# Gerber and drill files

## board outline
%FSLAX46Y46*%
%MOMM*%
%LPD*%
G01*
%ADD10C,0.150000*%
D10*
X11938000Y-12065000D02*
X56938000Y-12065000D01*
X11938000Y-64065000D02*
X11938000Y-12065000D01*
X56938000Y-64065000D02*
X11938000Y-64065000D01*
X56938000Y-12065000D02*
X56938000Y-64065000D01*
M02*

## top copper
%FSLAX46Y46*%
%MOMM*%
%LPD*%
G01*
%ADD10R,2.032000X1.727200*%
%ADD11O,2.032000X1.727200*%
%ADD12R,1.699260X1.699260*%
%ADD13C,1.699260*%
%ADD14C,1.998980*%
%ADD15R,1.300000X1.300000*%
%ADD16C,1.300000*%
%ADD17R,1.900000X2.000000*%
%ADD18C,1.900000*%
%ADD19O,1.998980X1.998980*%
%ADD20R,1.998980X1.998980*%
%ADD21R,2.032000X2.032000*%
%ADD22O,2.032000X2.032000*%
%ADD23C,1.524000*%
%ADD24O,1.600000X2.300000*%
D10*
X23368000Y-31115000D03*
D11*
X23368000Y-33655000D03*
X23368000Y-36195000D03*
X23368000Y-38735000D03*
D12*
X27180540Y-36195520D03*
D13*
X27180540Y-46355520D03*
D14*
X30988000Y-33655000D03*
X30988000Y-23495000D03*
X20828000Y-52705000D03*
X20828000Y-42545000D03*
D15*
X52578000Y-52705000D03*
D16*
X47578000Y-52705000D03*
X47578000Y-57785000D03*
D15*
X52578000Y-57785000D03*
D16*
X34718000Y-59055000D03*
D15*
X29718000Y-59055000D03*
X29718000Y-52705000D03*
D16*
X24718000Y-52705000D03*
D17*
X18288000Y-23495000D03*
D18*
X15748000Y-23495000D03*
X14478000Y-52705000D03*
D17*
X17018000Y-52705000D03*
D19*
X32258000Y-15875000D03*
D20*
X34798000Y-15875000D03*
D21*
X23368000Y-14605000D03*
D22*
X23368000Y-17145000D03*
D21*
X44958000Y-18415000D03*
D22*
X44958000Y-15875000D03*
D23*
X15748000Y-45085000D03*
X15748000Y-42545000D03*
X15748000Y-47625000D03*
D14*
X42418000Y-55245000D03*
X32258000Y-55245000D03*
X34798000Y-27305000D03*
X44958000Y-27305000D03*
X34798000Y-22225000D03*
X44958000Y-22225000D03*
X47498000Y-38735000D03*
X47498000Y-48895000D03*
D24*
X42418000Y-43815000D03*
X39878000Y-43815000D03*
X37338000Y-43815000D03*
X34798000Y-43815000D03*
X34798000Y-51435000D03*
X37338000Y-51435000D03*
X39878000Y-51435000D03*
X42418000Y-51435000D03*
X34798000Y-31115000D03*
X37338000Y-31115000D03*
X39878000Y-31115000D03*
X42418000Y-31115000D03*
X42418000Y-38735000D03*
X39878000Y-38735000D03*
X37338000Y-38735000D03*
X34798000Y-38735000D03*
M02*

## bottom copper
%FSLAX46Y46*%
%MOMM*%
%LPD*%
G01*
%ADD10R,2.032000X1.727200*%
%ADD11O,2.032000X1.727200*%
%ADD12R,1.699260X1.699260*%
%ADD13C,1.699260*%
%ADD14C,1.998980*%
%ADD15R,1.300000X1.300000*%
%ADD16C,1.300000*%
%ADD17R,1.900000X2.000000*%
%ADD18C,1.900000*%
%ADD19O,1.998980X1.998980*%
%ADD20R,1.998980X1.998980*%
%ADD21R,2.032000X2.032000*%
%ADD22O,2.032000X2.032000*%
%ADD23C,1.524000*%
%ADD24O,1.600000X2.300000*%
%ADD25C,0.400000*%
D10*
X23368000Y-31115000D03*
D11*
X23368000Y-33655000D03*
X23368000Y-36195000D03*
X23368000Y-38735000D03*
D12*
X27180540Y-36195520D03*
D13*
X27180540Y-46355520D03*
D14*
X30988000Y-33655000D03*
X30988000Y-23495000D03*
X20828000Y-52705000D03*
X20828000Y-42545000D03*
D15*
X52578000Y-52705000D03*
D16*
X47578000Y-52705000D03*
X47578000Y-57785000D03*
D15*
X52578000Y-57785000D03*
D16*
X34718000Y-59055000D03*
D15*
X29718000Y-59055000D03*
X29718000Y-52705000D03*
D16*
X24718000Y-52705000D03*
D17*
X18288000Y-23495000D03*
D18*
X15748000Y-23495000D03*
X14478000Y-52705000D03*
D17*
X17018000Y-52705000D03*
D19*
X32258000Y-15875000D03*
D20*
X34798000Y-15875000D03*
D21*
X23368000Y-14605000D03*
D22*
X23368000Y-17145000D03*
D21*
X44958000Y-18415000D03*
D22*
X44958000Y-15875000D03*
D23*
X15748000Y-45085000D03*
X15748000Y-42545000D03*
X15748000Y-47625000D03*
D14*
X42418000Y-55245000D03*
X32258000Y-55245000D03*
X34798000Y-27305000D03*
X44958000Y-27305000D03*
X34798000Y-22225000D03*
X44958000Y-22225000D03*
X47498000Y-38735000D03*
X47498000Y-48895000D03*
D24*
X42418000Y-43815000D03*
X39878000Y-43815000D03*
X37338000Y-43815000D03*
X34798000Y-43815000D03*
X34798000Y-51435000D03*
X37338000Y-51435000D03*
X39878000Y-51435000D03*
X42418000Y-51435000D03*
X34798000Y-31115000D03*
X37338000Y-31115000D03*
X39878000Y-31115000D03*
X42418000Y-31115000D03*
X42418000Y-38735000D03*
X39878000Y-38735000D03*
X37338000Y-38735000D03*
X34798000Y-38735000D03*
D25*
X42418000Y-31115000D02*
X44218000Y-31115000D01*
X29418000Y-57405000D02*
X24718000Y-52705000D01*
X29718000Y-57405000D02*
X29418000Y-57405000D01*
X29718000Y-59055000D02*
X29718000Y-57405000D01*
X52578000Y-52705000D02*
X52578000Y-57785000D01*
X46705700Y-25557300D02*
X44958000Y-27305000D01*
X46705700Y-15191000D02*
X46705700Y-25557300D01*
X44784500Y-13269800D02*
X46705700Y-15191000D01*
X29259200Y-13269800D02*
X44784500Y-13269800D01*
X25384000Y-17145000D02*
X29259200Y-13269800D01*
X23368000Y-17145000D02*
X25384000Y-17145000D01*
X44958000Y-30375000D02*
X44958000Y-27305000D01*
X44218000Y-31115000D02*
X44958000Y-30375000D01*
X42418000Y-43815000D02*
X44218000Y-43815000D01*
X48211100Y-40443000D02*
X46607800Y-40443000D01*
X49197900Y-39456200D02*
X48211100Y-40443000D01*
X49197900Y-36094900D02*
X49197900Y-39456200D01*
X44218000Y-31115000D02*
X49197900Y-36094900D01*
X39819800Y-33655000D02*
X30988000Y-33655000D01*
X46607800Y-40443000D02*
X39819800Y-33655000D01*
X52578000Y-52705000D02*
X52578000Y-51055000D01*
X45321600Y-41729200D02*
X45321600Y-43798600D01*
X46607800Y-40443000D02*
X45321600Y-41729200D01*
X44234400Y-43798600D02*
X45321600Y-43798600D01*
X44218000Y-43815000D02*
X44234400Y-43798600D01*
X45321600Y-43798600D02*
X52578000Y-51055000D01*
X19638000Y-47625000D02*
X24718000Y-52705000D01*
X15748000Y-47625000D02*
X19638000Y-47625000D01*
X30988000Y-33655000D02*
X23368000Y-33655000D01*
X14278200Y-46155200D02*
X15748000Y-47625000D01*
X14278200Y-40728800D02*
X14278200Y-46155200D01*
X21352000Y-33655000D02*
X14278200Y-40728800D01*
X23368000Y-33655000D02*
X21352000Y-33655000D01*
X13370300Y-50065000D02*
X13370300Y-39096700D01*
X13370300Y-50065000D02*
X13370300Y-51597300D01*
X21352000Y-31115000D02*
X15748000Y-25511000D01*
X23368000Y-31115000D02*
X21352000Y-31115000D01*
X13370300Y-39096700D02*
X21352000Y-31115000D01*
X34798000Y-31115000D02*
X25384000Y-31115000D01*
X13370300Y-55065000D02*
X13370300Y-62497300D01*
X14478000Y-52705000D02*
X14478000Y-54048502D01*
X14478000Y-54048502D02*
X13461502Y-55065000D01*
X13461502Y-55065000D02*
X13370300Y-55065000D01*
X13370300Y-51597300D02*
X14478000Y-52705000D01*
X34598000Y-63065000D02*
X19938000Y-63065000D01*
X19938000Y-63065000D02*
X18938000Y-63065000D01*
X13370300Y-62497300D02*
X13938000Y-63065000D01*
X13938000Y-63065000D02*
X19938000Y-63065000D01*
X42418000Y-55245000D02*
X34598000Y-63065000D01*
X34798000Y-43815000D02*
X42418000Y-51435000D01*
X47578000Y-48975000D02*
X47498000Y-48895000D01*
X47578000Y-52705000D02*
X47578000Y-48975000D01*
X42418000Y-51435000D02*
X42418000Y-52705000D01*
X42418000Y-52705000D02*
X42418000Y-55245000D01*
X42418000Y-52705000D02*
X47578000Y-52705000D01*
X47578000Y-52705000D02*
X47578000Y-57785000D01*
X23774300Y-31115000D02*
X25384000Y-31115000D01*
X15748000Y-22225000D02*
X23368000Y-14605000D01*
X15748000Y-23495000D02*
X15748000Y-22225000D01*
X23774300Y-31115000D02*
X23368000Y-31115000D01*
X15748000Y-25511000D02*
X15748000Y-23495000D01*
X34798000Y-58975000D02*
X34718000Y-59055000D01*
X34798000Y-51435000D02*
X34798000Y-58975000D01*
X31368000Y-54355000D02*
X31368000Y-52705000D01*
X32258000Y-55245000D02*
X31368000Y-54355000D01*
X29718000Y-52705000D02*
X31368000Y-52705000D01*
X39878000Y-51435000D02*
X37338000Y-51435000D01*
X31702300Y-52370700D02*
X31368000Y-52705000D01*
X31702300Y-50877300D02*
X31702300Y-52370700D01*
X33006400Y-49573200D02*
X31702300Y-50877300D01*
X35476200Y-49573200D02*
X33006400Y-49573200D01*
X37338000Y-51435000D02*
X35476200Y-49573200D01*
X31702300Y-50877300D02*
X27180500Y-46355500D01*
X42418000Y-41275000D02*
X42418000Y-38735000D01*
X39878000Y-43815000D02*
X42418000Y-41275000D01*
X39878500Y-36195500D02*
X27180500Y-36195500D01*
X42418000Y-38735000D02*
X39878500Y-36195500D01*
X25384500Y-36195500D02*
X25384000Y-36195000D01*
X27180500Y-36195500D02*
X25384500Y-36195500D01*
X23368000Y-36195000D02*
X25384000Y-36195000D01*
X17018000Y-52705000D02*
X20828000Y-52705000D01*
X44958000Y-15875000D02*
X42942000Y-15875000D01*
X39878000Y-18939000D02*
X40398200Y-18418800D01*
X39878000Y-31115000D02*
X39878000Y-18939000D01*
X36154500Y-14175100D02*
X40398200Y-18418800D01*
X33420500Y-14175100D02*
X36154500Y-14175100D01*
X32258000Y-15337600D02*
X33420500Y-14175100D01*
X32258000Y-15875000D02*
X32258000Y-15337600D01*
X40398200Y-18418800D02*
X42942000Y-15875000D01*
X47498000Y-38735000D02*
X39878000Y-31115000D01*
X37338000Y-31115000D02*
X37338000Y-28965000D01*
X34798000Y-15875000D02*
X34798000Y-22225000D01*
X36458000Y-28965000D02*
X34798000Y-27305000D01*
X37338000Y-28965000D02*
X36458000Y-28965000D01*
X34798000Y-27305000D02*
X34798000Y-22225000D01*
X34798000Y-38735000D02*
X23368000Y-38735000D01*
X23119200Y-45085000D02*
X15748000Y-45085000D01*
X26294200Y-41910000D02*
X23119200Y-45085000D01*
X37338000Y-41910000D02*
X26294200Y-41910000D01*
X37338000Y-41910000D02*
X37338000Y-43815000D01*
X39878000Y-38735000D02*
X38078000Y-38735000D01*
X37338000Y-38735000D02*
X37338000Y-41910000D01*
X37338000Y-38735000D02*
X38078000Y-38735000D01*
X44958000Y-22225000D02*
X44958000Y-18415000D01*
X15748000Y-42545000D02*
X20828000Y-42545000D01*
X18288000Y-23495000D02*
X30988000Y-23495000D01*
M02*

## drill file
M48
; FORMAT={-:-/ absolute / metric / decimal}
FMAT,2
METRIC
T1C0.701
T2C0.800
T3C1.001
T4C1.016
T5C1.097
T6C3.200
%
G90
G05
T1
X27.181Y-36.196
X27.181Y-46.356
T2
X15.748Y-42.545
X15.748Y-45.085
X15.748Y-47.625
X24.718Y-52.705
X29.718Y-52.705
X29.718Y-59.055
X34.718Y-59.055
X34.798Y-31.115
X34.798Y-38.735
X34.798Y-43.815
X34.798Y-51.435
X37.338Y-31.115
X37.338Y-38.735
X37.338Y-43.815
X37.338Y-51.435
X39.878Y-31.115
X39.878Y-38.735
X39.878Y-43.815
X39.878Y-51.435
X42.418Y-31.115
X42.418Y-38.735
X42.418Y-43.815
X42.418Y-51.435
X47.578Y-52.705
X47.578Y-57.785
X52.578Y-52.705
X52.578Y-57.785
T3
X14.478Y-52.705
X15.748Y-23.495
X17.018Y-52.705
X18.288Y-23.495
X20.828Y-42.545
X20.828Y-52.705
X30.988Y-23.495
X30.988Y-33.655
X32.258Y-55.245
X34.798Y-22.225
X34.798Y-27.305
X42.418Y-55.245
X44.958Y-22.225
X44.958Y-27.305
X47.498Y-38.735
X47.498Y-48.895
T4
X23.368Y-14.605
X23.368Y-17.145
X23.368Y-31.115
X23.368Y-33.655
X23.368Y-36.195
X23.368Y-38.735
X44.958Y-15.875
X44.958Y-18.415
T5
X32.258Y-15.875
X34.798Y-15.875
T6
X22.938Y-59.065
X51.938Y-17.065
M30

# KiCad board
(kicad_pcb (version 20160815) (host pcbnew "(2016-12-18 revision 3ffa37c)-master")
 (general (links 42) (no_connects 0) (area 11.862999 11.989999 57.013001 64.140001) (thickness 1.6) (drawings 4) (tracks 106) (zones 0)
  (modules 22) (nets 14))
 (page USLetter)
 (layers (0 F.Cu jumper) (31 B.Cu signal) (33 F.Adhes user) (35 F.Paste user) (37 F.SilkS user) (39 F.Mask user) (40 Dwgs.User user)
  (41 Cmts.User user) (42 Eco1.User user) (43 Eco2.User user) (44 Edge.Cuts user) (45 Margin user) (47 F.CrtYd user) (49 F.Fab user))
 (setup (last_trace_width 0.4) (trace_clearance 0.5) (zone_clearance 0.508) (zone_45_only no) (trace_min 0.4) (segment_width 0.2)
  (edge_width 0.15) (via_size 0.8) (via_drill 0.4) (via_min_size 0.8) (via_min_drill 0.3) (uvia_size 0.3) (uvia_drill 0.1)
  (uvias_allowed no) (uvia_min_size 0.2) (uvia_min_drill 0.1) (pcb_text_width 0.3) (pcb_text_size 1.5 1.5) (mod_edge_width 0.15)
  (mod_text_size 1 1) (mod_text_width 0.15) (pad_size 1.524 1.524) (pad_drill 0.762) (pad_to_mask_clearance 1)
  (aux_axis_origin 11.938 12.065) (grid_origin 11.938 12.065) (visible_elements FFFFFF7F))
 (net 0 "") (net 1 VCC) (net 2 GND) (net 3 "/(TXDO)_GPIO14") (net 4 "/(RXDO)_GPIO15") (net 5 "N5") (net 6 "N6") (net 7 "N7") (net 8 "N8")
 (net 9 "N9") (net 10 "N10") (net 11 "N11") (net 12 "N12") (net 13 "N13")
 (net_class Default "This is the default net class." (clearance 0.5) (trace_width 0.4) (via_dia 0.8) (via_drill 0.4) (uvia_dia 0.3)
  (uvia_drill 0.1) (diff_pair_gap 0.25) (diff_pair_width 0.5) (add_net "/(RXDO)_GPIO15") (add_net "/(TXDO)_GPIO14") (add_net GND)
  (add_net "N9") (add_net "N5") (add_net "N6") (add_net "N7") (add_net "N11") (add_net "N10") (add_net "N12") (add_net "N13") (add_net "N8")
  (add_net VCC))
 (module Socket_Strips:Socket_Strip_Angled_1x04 (layer F.Cu) (at 23.368 31.115 270)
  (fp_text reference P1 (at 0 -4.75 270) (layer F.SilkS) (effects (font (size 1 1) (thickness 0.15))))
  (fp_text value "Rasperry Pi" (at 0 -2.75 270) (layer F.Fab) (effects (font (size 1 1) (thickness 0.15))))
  (pad 1 thru_hole rect (at 0 0 270) (size 1.7272 2.032) (drill 1.016) (layers *.Cu *.Mask) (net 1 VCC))
  (pad 2 thru_hole oval (at 2.54 0 270) (size 1.7272 2.032) (drill 1.016) (layers *.Cu *.Mask) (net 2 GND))
  (pad 3 thru_hole oval (at 5.08 0 270) (size 1.7272 2.032) (drill 1.016) (layers *.Cu *.Mask) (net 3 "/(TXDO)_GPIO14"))
  (pad 4 thru_hole oval (at 7.62 0 270) (size 1.7272 2.032) (drill 1.016) (layers *.Cu *.Mask) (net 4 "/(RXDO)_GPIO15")))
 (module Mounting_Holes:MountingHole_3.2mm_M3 (layer F.Cu) (at 22.938 59.065)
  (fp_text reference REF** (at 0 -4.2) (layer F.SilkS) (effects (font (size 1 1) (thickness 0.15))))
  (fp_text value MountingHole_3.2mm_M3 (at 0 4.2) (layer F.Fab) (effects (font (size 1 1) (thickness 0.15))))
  (pad 1 np_thru_hole circle (at 0 0) (size 3.2 3.2) (drill 3.2) (layers *.Cu *.Mask)))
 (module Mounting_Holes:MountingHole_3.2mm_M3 (layer F.Cu) (at 51.938 17.065)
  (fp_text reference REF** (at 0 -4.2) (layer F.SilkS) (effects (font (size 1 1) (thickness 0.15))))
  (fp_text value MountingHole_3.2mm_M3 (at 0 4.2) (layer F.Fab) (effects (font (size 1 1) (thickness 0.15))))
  (pad 1 np_thru_hole circle (at 0 0) (size 3.2 3.2) (drill 3.2) (layers *.Cu *.Mask)))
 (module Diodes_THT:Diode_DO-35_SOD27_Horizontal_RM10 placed (layer F.Cu) (at 27.178 36.195 270)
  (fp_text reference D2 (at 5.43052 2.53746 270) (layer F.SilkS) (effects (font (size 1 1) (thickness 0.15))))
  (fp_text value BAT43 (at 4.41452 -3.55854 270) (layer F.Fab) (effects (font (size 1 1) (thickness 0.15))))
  (pad 1 thru_hole rect (at 0.00052 -0.00254 90) (size 1.69926 1.69926) (drill 0.70104) (layers *.Cu *.Mask) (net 3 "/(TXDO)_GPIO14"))
  (pad 2 thru_hole circle (at 10.16052 -0.00254 90) (size 1.69926 1.69926) (drill 0.70104) (layers *.Cu *.Mask) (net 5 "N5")))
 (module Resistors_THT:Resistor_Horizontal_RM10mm (layer F.Cu) (at 30.988 23.495 270)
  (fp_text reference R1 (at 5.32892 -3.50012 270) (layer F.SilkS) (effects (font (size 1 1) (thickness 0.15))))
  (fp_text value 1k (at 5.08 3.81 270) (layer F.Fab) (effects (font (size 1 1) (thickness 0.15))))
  (pad 2 thru_hole circle (at 10.16 0 270) (size 1.99898 1.99898) (drill 1.00076) (layers *.Cu *.SilkS *.Mask) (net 2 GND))
  (pad 1 thru_hole circle (at 0 0 270) (size 1.99898 1.99898) (drill 1.00076) (layers *.Cu *.SilkS *.Mask) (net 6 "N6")))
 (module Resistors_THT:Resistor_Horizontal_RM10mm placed (layer F.Cu) (at 20.828 42.545 270)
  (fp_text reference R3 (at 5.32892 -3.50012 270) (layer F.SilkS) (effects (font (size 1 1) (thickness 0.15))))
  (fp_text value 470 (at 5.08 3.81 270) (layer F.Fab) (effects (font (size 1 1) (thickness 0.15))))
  (pad 2 thru_hole circle (at 10.16 0 270) (size 1.99898 1.99898) (drill 1.00076) (layers *.Cu *.SilkS *.Mask) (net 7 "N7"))
  (pad 1 thru_hole circle (at 0 0 270) (size 1.99898 1.99898) (drill 1.00076) (layers *.Cu *.SilkS *.Mask) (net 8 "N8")))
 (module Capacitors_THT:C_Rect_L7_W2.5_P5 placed (layer F.Cu) (at 52.578 52.705 180)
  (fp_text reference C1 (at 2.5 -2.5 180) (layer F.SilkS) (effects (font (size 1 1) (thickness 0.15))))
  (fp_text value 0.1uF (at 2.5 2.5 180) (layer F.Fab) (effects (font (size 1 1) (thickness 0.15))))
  (pad 1 thru_hole rect (at 0 0 180) (size 1.3 1.3) (drill 0.8) (layers *.Cu *.Mask) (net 2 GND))
  (pad 2 thru_hole circle (at 5 0 180) (size 1.3 1.3) (drill 0.8) (layers *.Cu *.Mask) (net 1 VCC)))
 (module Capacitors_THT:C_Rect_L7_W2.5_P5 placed (layer F.Cu) (at 52.578 57.785 180)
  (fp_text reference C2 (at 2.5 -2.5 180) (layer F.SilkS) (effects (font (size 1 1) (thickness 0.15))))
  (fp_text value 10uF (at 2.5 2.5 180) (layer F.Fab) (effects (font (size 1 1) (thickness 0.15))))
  (pad 2 thru_hole circle (at 5 0 180) (size 1.3 1.3) (drill 0.8) (layers *.Cu *.Mask) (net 1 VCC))
  (pad 1 thru_hole rect (at 0 0 180) (size 1.3 1.3) (drill 0.8) (layers *.Cu *.Mask) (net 2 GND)))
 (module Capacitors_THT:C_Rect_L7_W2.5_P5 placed (layer F.Cu) (at 29.718 59.055)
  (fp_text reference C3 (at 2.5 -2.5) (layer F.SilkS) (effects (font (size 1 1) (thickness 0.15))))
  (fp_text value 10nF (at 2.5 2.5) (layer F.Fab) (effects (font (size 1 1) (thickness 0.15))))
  (pad 2 thru_hole circle (at 5 0) (size 1.3 1.3) (drill 0.8) (layers *.Cu *.Mask) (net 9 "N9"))
  (pad 1 thru_hole rect (at 0 0) (size 1.3 1.3) (drill 0.8) (layers *.Cu *.Mask) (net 2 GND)))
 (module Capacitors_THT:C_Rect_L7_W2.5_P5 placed (layer F.Cu) (at 29.718 52.705 180)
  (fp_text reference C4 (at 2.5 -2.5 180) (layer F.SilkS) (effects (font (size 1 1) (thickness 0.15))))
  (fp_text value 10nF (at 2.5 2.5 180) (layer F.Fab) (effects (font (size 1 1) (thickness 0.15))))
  (pad 1 thru_hole rect (at 0 0 180) (size 1.3 1.3) (drill 0.8) (layers *.Cu *.Mask) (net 5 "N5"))
  (pad 2 thru_hole circle (at 5 0 180) (size 1.3 1.3) (drill 0.8) (layers *.Cu *.Mask) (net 2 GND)))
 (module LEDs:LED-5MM (layer F.Cu) (at 18.288 23.495 180)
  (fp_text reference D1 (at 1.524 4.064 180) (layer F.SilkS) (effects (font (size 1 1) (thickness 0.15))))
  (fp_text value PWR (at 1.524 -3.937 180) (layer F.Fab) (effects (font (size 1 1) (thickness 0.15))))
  (pad 1 thru_hole rect (at 0 0 270) (size 2 1.9) (drill 1.00076) (layers *.Cu *.Mask) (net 6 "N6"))
  (pad 2 thru_hole circle (at 2.54 0 180) (size 1.9 1.9) (drill 1.00076) (layers *.Cu *.Mask) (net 1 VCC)))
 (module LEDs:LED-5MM (layer F.Cu) (at 17.018 52.705 180)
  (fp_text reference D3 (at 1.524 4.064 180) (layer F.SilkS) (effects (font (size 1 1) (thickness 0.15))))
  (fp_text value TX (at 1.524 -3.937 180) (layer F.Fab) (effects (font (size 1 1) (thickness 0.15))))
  (pad 2 thru_hole circle (at 2.54 0 180) (size 1.9 1.9) (drill 1.00076) (layers *.Cu *.Mask) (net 1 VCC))
  (pad 1 thru_hole rect (at 0 0 270) (size 2 1.9) (drill 1.00076) (layers *.Cu *.Mask) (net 7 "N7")))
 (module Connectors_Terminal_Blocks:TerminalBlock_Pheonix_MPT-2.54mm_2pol (layer F.Cu) (at 34.798 15.875 180)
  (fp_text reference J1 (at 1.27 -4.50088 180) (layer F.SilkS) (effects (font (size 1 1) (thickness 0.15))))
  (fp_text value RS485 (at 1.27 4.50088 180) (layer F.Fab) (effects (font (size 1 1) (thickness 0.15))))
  (pad 2 thru_hole oval (at 2.54 0 180) (size 1.99898 1.99898) (drill 1.09728) (layers *.Cu *.Mask) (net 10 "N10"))
  (pad 1 thru_hole rect (at 0 0 180) (size 1.99898 1.99898) (drill 1.09728) (layers *.Cu *.Mask) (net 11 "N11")))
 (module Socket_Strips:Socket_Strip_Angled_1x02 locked (layer F.Cu) (at 23.368 14.605 270)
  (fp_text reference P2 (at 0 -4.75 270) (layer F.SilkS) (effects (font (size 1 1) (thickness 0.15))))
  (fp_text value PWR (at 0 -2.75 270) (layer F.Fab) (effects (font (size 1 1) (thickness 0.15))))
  (pad 1 thru_hole rect (at 0 0 270) (size 2.032 2.032) (drill 1.016) (layers *.Cu *.Mask) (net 1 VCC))
  (pad 2 thru_hole oval (at 2.54 0 270) (size 2.032 2.032) (drill 1.016) (layers *.Cu *.Mask) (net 2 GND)))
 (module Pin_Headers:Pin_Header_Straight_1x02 (layer F.Cu) (at 44.958 18.415 180)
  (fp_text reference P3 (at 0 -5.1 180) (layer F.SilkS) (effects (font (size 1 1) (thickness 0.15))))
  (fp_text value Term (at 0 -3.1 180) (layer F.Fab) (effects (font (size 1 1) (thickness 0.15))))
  (pad 1 thru_hole rect (at 0 0 180) (size 2.032 2.032) (drill 1.016) (layers *.Cu *.Mask) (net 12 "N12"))
  (pad 2 thru_hole oval (at 0 2.54 180) (size 2.032 2.032) (drill 1.016) (layers *.Cu *.Mask) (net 10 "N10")))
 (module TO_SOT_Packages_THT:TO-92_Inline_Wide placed (layer F.Cu) (at 15.748 47.625 90)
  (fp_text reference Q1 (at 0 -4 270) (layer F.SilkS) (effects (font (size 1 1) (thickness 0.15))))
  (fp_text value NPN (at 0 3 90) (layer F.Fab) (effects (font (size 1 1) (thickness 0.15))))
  (pad 2 thru_hole circle (at 2.54 0 180) (size 1.524 1.524) (drill 0.8) (layers *.Cu *.Mask) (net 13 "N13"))
  (pad 3 thru_hole circle (at 5.08 0 180) (size 1.524 1.524) (drill 0.8) (layers *.Cu *.Mask) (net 8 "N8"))
  (pad 1 thru_hole circle (at 0 0 180) (size 1.524 1.524) (drill 0.8) (layers *.Cu *.Mask) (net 2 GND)))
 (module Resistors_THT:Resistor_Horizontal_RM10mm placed (layer F.Cu) (at 32.258 55.245)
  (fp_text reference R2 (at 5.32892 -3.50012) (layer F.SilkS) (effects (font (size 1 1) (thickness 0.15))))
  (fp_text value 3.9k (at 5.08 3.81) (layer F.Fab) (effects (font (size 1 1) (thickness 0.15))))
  (pad 2 thru_hole circle (at 10.16 0) (size 1.99898 1.99898) (drill 1.00076) (layers *.Cu *.SilkS *.Mask) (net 1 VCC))
  (pad 1 thru_hole circle (at 0 0) (size 1.99898 1.99898) (drill 1.00076) (layers *.Cu *.SilkS *.Mask) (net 5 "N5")))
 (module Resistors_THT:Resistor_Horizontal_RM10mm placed (layer F.Cu) (at 44.958 27.305 180)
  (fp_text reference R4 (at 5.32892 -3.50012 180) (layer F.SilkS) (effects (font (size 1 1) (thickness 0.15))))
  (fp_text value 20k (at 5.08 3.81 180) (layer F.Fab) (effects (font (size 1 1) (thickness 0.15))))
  (pad 2 thru_hole circle (at 10.16 0 180) (size 1.99898 1.99898) (drill 1.00076) (layers *.Cu *.SilkS *.Mask) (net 11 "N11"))
  (pad 1 thru_hole circle (at 0 0 180) (size 1.99898 1.99898) (drill 1.00076) (layers *.Cu *.SilkS *.Mask) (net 2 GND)))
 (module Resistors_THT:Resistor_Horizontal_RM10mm (layer F.Cu) (at 34.798 22.225)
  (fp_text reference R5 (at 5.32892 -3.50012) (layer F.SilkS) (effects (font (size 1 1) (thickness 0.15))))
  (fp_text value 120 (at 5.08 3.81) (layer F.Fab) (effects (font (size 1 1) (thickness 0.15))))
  (pad 1 thru_hole circle (at 0 0) (size 1.99898 1.99898) (drill 1.00076) (layers *.Cu *.SilkS *.Mask) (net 11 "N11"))
  (pad 2 thru_hole circle (at 10.16 0) (size 1.99898 1.99898) (drill 1.00076) (layers *.Cu *.SilkS *.Mask) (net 12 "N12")))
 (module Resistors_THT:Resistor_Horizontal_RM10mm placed (layer F.Cu) (at 47.498 38.735 270)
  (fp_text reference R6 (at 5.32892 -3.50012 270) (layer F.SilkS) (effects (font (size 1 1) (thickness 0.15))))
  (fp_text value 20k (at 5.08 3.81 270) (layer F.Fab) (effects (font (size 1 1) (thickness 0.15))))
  (pad 1 thru_hole circle (at 0 0 270) (size 1.99898 1.99898) (drill 1.00076) (layers *.Cu *.SilkS *.Mask) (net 10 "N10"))
  (pad 2 thru_hole circle (at 10.16 0 270) (size 1.99898 1.99898) (drill 1.00076) (layers *.Cu *.SilkS *.Mask) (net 1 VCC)))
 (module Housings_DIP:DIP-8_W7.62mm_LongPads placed (layer F.Cu) (at 42.418 43.815 270)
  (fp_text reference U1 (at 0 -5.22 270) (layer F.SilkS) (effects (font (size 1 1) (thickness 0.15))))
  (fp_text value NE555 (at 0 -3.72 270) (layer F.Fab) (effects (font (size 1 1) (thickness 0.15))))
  (pad 1 thru_hole oval (at 0 0 270) (size 2.3 1.6) (drill 0.8) (layers *.Cu *.Mask) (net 2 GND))
  (pad 2 thru_hole oval (at 0 2.54 270) (size 2.3 1.6) (drill 0.8) (layers *.Cu *.Mask) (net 3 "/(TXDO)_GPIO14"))
  (pad 3 thru_hole oval (at 0 5.08 270) (size 2.3 1.6) (drill 0.8) (layers *.Cu *.Mask) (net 13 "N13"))
  (pad 4 thru_hole oval (at 0 7.62 270) (size 2.3 1.6) (drill 0.8) (layers *.Cu *.Mask) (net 1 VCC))
  (pad 5 thru_hole oval (at 7.62 7.62 270) (size 2.3 1.6) (drill 0.8) (layers *.Cu *.Mask) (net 9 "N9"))
  (pad 6 thru_hole oval (at 7.62 5.08 270) (size 2.3 1.6) (drill 0.8) (layers *.Cu *.Mask) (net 5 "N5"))
  (pad 7 thru_hole oval (at 7.62 2.54 270) (size 2.3 1.6) (drill 0.8) (layers *.Cu *.Mask) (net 5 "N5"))
  (pad 8 thru_hole oval (at 7.62 0 270) (size 2.3 1.6) (drill 0.8) (layers *.Cu *.Mask) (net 1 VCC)))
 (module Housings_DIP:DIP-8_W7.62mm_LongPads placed (layer F.Cu) (at 34.798 38.735 90)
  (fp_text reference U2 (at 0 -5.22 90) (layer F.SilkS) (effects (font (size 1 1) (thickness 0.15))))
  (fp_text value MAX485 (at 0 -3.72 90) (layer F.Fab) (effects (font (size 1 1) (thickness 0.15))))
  (pad 8 thru_hole oval (at 7.62 0 90) (size 2.3 1.6) (drill 0.8) (layers *.Cu *.Mask) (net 1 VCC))
  (pad 7 thru_hole oval (at 7.62 2.54 90) (size 2.3 1.6) (drill 0.8) (layers *.Cu *.Mask) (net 11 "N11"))
  (pad 6 thru_hole oval (at 7.62 5.08 90) (size 2.3 1.6) (drill 0.8) (layers *.Cu *.Mask) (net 10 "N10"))
  (pad 5 thru_hole oval (at 7.62 7.62 90) (size 2.3 1.6) (drill 0.8) (layers *.Cu *.Mask) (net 2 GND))
  (pad 4 thru_hole oval (at 0 7.62 90) (size 2.3 1.6) (drill 0.8) (layers *.Cu *.Mask) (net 3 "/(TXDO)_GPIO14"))
  (pad 3 thru_hole oval (at 0 5.08 90) (size 2.3 1.6) (drill 0.8) (layers *.Cu *.Mask) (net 13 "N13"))
  (pad 2 thru_hole oval (at 0 2.54 90) (size 2.3 1.6) (drill 0.8) (layers *.Cu *.Mask) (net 13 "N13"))
  (pad 1 thru_hole oval (at 0 0 90) (size 2.3 1.6) (drill 0.8) (layers *.Cu *.Mask) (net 4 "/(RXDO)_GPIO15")))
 (gr_line (start 11.938 12.065) (end 56.938 12.065) (layer Edge.Cuts) (width 0.15))
 (gr_line (start 11.938 64.065) (end 11.938 12.065) (layer Edge.Cuts) (width 0.15))
 (gr_line (start 56.938 64.065) (end 11.938 64.065) (layer Edge.Cuts) (width 0.15))
 (gr_line (start 56.938 12.065) (end 56.938 64.065) (layer Edge.Cuts) (width 0.15))
 (segment (start 42.418 31.115) (end 44.218 31.115) (width 0.4) (layer B.Cu) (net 2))
 (segment (start 29.418 57.405) (end 24.718 52.705) (width 0.4) (layer B.Cu) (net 2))
 (segment (start 29.718 57.405) (end 29.418 57.405) (width 0.4) (layer B.Cu) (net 2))
 (segment (start 29.718 59.055) (end 29.718 57.405) (width 0.4) (layer B.Cu) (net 2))
 (segment (start 52.578 52.705) (end 52.578 57.785) (width 0.4) (layer B.Cu) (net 2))
 (segment (start 46.7057 25.5573) (end 44.958 27.305) (width 0.4) (layer B.Cu) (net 2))
 (segment (start 46.7057 15.191) (end 46.7057 25.5573) (width 0.4) (layer B.Cu) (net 2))
 (segment (start 44.7845 13.2698) (end 46.7057 15.191) (width 0.4) (layer B.Cu) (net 2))
 (segment (start 29.2592 13.2698) (end 44.7845 13.2698) (width 0.4) (layer B.Cu) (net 2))
 (segment (start 25.384 17.145) (end 29.2592 13.2698) (width 0.4) (layer B.Cu) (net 2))
 (segment (start 23.368 17.145) (end 25.384 17.145) (width 0.4) (layer B.Cu) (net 2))
 (segment (start 44.958 30.375) (end 44.958 27.305) (width 0.4) (layer B.Cu) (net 2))
 (segment (start 44.218 31.115) (end 44.958 30.375) (width 0.4) (layer B.Cu) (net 2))
 (segment (start 42.418 43.815) (end 44.218 43.815) (width 0.4) (layer B.Cu) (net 2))
 (segment (start 48.2111 40.443) (end 46.6078 40.443) (width 0.4) (layer B.Cu) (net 2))
 (segment (start 49.1979 39.4562) (end 48.2111 40.443) (width 0.4) (layer B.Cu) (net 2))
 (segment (start 49.1979 36.0949) (end 49.1979 39.4562) (width 0.4) (layer B.Cu) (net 2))
 (segment (start 44.218 31.115) (end 49.1979 36.0949) (width 0.4) (layer B.Cu) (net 2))
 (segment (start 39.8198 33.655) (end 30.988 33.655) (width 0.4) (layer B.Cu) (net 2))
 (segment (start 46.6078 40.443) (end 39.8198 33.655) (width 0.4) (layer B.Cu) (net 2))
 (segment (start 52.578 52.705) (end 52.578 51.055) (width 0.4) (layer B.Cu) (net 2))
 (segment (start 45.3216 41.7292) (end 45.3216 43.7986) (width 0.4) (layer B.Cu) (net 2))
 (segment (start 46.6078 40.443) (end 45.3216 41.7292) (width 0.4) (layer B.Cu) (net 2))
 (segment (start 44.2344 43.7986) (end 45.3216 43.7986) (width 0.4) (layer B.Cu) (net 2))
 (segment (start 44.218 43.815) (end 44.2344 43.7986) (width 0.4) (layer B.Cu) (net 2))
 (segment (start 45.3216 43.7986) (end 52.578 51.055) (width 0.4) (layer B.Cu) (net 2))
 (segment (start 19.638 47.625) (end 24.718 52.705) (width 0.4) (layer B.Cu) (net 2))
 (segment (start 15.748 47.625) (end 19.638 47.625) (width 0.4) (layer B.Cu) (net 2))
 (segment (start 30.988 33.655) (end 23.368 33.655) (width 0.4) (layer B.Cu) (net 2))
 (segment (start 14.2782 46.1552) (end 15.748 47.625) (width 0.4) (layer B.Cu) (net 2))
 (segment (start 14.2782 40.7288) (end 14.2782 46.1552) (width 0.4) (layer B.Cu) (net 2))
 (segment (start 21.352 33.655) (end 14.2782 40.7288) (width 0.4) (layer B.Cu) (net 2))
 (segment (start 23.368 33.655) (end 21.352 33.655) (width 0.4) (layer B.Cu) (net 2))
 (segment (start 13.3703 50.065) (end 13.3703 39.0967) (width 0.4) (layer B.Cu) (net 1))
 (segment (start 13.3703 50.065) (end 13.3703 51.5973) (width 0.4) (layer B.Cu) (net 1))
 (segment (start 21.352 31.115) (end 15.748 25.511) (width 0.4) (layer B.Cu) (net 1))
 (segment (start 23.368 31.115) (end 21.352 31.115) (width 0.4) (layer B.Cu) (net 1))
 (segment (start 13.3703 39.0967) (end 21.352 31.115) (width 0.4) (layer B.Cu) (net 1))
 (segment (start 34.798 31.115) (end 25.384 31.115) (width 0.4) (layer B.Cu) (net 1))
 (segment (start 13.3703 55.065) (end 13.3703 62.4973) (width 0.4) (layer B.Cu) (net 1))
 (segment (start 14.478 52.705) (end 14.478 54.048502) (width 0.4) (layer B.Cu) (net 1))
 (segment (start 14.478 54.048502) (end 13.461502 55.065) (width 0.4) (layer B.Cu) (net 1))
 (segment (start 13.461502 55.065) (end 13.3703 55.065) (width 0.4) (layer B.Cu) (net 1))
 (segment (start 13.3703 51.5973) (end 14.478 52.705) (width 0.4) (layer B.Cu) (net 1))
 (segment (start 34.598 63.065) (end 19.938 63.065) (width 0.4) (layer B.Cu) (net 1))
 (segment (start 19.938 63.065) (end 18.938 63.065) (width 0.4) (layer B.Cu) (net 1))
 (segment (start 13.3703 62.4973) (end 13.938 63.065) (width 0.4) (layer B.Cu) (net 1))
 (segment (start 13.938 63.065) (end 19.938 63.065) (width 0.4) (layer B.Cu) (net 1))
 (segment (start 42.418 55.245) (end 34.598 63.065) (width 0.4) (layer B.Cu) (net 1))
 (segment (start 34.798 43.815) (end 42.418 51.435) (width 0.4) (layer B.Cu) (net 1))
 (segment (start 47.578 48.975) (end 47.498 48.895) (width 0.4) (layer B.Cu) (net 1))
 (segment (start 47.578 52.705) (end 47.578 48.975) (width 0.4) (layer B.Cu) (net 1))
 (segment (start 42.418 51.435) (end 42.418 52.705) (width 0.4) (layer B.Cu) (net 1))
 (segment (start 42.418 52.705) (end 42.418 55.245) (width 0.4) (layer B.Cu) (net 1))
 (segment (start 42.418 52.705) (end 47.578 52.705) (width 0.4) (layer B.Cu) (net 1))
 (segment (start 47.578 52.705) (end 47.578 57.785) (width 0.4) (layer B.Cu) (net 1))
 (segment (start 23.7743 31.115) (end 25.384 31.115) (width 0.4) (layer B.Cu) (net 1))
 (segment (start 15.748 22.225) (end 23.368 14.605) (width 0.4) (layer B.Cu) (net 1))
 (segment (start 15.748 23.495) (end 15.748 22.225) (width 0.4) (layer B.Cu) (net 1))
 (segment (start 23.7743 31.115) (end 23.368 31.115) (width 0.4) (layer B.Cu) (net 1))
 (segment (start 15.748 25.511) (end 15.748 23.495) (width 0.4) (layer B.Cu) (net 1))
 (segment (start 34.798 58.975) (end 34.718 59.055) (width 0.4) (layer B.Cu) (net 9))
 (segment (start 34.798 51.435) (end 34.798 58.975) (width 0.4) (layer B.Cu) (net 9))
 (segment (start 31.368 54.355) (end 31.368 52.705) (width 0.4) (layer B.Cu) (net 5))
 (segment (start 32.258 55.245) (end 31.368 54.355) (width 0.4) (layer B.Cu) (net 5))
 (segment (start 29.718 52.705) (end 31.368 52.705) (width 0.4) (layer B.Cu) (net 5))
 (segment (start 39.878 51.435) (end 37.338 51.435) (width 0.4) (layer B.Cu) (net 5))
 (segment (start 31.7023 52.3707) (end 31.368 52.705) (width 0.4) (layer B.Cu) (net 5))
 (segment (start 31.7023 50.8773) (end 31.7023 52.3707) (width 0.4) (layer B.Cu) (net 5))
 (segment (start 33.0064 49.5732) (end 31.7023 50.8773) (width 0.4) (layer B.Cu) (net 5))
 (segment (start 35.4762 49.5732) (end 33.0064 49.5732) (width 0.4) (layer B.Cu) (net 5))
 (segment (start 37.338 51.435) (end 35.4762 49.5732) (width 0.4) (layer B.Cu) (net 5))
 (segment (start 31.7023 50.8773) (end 27.1805 46.3555) (width 0.4) (layer B.Cu) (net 5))
 (segment (start 42.418 41.275) (end 42.418 38.735) (width 0.4) (layer B.Cu) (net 3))
 (segment (start 39.878 43.815) (end 42.418 41.275) (width 0.4) (layer B.Cu) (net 3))
 (segment (start 39.8785 36.1955) (end 27.1805 36.1955) (width 0.4) (layer B.Cu) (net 3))
 (segment (start 42.418 38.735) (end 39.8785 36.1955) (width 0.4) (layer B.Cu) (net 3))
 (segment (start 25.3845 36.1955) (end 25.384 36.195) (width 0.4) (layer B.Cu) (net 3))
 (segment (start 27.1805 36.1955) (end 25.3845 36.1955) (width 0.4) (layer B.Cu) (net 3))
 (segment (start 23.368 36.195) (end 25.384 36.195) (width 0.4) (layer B.Cu) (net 3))
 (segment (start 17.018 52.705) (end 20.828 52.705) (width 0.4) (layer B.Cu) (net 7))
 (segment (start 44.958 15.875) (end 42.942 15.875) (width 0.4) (layer B.Cu) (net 10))
 (segment (start 39.878 18.939) (end 40.3982 18.4188) (width 0.4) (layer B.Cu) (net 10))
 (segment (start 39.878 31.115) (end 39.878 18.939) (width 0.4) (layer B.Cu) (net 10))
 (segment (start 36.1545 14.1751) (end 40.3982 18.4188) (width 0.4) (layer B.Cu) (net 10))
 (segment (start 33.4205 14.1751) (end 36.1545 14.1751) (width 0.4) (layer B.Cu) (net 10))
 (segment (start 32.258 15.3376) (end 33.4205 14.1751) (width 0.4) (layer B.Cu) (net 10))
 (segment (start 32.258 15.875) (end 32.258 15.3376) (width 0.4) (layer B.Cu) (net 10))
 (segment (start 40.3982 18.4188) (end 42.942 15.875) (width 0.4) (layer B.Cu) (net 10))
 (segment (start 47.498 38.735) (end 39.878 31.115) (width 0.4) (layer B.Cu) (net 10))
 (segment (start 37.338 31.115) (end 37.338 28.965) (width 0.4) (layer B.Cu) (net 11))
 (segment (start 34.798 15.875) (end 34.798 22.225) (width 0.4) (layer B.Cu) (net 11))
 (segment (start 36.458 28.965) (end 34.798 27.305) (width 0.4) (layer B.Cu) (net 11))
 (segment (start 37.338 28.965) (end 36.458 28.965) (width 0.4) (layer B.Cu) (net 11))
 (segment (start 34.798 27.305) (end 34.798 22.225) (width 0.4) (layer B.Cu) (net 11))
 (segment (start 34.798 38.735) (end 23.368 38.735) (width 0.4) (layer B.Cu) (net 4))
 (segment (start 23.1192 45.085) (end 15.748 45.085) (width 0.4) (layer B.Cu) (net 13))
 (segment (start 26.2942 41.91) (end 23.1192 45.085) (width 0.4) (layer B.Cu) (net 13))
 (segment (start 37.338 41.91) (end 26.2942 41.91) (width 0.4) (layer B.Cu) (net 13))
 (segment (start 37.338 41.91) (end 37.338 43.815) (width 0.4) (layer B.Cu) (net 13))
 (segment (start 39.878 38.735) (end 38.078 38.735) (width 0.4) (layer B.Cu) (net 13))
 (segment (start 37.338 38.735) (end 37.338 41.91) (width 0.4) (layer B.Cu) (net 13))
 (segment (start 37.338 38.735) (end 38.078 38.735) (width 0.4) (layer B.Cu) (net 13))
 (segment (start 44.958 22.225) (end 44.958 18.415) (width 0.4) (layer B.Cu) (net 12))
 (segment (start 15.748 42.545) (end 20.828 42.545) (width 0.4) (layer B.Cu) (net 8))
 (segment (start 18.288 23.495) (end 30.988 23.495) (width 0.4) (layer B.Cu) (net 6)))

